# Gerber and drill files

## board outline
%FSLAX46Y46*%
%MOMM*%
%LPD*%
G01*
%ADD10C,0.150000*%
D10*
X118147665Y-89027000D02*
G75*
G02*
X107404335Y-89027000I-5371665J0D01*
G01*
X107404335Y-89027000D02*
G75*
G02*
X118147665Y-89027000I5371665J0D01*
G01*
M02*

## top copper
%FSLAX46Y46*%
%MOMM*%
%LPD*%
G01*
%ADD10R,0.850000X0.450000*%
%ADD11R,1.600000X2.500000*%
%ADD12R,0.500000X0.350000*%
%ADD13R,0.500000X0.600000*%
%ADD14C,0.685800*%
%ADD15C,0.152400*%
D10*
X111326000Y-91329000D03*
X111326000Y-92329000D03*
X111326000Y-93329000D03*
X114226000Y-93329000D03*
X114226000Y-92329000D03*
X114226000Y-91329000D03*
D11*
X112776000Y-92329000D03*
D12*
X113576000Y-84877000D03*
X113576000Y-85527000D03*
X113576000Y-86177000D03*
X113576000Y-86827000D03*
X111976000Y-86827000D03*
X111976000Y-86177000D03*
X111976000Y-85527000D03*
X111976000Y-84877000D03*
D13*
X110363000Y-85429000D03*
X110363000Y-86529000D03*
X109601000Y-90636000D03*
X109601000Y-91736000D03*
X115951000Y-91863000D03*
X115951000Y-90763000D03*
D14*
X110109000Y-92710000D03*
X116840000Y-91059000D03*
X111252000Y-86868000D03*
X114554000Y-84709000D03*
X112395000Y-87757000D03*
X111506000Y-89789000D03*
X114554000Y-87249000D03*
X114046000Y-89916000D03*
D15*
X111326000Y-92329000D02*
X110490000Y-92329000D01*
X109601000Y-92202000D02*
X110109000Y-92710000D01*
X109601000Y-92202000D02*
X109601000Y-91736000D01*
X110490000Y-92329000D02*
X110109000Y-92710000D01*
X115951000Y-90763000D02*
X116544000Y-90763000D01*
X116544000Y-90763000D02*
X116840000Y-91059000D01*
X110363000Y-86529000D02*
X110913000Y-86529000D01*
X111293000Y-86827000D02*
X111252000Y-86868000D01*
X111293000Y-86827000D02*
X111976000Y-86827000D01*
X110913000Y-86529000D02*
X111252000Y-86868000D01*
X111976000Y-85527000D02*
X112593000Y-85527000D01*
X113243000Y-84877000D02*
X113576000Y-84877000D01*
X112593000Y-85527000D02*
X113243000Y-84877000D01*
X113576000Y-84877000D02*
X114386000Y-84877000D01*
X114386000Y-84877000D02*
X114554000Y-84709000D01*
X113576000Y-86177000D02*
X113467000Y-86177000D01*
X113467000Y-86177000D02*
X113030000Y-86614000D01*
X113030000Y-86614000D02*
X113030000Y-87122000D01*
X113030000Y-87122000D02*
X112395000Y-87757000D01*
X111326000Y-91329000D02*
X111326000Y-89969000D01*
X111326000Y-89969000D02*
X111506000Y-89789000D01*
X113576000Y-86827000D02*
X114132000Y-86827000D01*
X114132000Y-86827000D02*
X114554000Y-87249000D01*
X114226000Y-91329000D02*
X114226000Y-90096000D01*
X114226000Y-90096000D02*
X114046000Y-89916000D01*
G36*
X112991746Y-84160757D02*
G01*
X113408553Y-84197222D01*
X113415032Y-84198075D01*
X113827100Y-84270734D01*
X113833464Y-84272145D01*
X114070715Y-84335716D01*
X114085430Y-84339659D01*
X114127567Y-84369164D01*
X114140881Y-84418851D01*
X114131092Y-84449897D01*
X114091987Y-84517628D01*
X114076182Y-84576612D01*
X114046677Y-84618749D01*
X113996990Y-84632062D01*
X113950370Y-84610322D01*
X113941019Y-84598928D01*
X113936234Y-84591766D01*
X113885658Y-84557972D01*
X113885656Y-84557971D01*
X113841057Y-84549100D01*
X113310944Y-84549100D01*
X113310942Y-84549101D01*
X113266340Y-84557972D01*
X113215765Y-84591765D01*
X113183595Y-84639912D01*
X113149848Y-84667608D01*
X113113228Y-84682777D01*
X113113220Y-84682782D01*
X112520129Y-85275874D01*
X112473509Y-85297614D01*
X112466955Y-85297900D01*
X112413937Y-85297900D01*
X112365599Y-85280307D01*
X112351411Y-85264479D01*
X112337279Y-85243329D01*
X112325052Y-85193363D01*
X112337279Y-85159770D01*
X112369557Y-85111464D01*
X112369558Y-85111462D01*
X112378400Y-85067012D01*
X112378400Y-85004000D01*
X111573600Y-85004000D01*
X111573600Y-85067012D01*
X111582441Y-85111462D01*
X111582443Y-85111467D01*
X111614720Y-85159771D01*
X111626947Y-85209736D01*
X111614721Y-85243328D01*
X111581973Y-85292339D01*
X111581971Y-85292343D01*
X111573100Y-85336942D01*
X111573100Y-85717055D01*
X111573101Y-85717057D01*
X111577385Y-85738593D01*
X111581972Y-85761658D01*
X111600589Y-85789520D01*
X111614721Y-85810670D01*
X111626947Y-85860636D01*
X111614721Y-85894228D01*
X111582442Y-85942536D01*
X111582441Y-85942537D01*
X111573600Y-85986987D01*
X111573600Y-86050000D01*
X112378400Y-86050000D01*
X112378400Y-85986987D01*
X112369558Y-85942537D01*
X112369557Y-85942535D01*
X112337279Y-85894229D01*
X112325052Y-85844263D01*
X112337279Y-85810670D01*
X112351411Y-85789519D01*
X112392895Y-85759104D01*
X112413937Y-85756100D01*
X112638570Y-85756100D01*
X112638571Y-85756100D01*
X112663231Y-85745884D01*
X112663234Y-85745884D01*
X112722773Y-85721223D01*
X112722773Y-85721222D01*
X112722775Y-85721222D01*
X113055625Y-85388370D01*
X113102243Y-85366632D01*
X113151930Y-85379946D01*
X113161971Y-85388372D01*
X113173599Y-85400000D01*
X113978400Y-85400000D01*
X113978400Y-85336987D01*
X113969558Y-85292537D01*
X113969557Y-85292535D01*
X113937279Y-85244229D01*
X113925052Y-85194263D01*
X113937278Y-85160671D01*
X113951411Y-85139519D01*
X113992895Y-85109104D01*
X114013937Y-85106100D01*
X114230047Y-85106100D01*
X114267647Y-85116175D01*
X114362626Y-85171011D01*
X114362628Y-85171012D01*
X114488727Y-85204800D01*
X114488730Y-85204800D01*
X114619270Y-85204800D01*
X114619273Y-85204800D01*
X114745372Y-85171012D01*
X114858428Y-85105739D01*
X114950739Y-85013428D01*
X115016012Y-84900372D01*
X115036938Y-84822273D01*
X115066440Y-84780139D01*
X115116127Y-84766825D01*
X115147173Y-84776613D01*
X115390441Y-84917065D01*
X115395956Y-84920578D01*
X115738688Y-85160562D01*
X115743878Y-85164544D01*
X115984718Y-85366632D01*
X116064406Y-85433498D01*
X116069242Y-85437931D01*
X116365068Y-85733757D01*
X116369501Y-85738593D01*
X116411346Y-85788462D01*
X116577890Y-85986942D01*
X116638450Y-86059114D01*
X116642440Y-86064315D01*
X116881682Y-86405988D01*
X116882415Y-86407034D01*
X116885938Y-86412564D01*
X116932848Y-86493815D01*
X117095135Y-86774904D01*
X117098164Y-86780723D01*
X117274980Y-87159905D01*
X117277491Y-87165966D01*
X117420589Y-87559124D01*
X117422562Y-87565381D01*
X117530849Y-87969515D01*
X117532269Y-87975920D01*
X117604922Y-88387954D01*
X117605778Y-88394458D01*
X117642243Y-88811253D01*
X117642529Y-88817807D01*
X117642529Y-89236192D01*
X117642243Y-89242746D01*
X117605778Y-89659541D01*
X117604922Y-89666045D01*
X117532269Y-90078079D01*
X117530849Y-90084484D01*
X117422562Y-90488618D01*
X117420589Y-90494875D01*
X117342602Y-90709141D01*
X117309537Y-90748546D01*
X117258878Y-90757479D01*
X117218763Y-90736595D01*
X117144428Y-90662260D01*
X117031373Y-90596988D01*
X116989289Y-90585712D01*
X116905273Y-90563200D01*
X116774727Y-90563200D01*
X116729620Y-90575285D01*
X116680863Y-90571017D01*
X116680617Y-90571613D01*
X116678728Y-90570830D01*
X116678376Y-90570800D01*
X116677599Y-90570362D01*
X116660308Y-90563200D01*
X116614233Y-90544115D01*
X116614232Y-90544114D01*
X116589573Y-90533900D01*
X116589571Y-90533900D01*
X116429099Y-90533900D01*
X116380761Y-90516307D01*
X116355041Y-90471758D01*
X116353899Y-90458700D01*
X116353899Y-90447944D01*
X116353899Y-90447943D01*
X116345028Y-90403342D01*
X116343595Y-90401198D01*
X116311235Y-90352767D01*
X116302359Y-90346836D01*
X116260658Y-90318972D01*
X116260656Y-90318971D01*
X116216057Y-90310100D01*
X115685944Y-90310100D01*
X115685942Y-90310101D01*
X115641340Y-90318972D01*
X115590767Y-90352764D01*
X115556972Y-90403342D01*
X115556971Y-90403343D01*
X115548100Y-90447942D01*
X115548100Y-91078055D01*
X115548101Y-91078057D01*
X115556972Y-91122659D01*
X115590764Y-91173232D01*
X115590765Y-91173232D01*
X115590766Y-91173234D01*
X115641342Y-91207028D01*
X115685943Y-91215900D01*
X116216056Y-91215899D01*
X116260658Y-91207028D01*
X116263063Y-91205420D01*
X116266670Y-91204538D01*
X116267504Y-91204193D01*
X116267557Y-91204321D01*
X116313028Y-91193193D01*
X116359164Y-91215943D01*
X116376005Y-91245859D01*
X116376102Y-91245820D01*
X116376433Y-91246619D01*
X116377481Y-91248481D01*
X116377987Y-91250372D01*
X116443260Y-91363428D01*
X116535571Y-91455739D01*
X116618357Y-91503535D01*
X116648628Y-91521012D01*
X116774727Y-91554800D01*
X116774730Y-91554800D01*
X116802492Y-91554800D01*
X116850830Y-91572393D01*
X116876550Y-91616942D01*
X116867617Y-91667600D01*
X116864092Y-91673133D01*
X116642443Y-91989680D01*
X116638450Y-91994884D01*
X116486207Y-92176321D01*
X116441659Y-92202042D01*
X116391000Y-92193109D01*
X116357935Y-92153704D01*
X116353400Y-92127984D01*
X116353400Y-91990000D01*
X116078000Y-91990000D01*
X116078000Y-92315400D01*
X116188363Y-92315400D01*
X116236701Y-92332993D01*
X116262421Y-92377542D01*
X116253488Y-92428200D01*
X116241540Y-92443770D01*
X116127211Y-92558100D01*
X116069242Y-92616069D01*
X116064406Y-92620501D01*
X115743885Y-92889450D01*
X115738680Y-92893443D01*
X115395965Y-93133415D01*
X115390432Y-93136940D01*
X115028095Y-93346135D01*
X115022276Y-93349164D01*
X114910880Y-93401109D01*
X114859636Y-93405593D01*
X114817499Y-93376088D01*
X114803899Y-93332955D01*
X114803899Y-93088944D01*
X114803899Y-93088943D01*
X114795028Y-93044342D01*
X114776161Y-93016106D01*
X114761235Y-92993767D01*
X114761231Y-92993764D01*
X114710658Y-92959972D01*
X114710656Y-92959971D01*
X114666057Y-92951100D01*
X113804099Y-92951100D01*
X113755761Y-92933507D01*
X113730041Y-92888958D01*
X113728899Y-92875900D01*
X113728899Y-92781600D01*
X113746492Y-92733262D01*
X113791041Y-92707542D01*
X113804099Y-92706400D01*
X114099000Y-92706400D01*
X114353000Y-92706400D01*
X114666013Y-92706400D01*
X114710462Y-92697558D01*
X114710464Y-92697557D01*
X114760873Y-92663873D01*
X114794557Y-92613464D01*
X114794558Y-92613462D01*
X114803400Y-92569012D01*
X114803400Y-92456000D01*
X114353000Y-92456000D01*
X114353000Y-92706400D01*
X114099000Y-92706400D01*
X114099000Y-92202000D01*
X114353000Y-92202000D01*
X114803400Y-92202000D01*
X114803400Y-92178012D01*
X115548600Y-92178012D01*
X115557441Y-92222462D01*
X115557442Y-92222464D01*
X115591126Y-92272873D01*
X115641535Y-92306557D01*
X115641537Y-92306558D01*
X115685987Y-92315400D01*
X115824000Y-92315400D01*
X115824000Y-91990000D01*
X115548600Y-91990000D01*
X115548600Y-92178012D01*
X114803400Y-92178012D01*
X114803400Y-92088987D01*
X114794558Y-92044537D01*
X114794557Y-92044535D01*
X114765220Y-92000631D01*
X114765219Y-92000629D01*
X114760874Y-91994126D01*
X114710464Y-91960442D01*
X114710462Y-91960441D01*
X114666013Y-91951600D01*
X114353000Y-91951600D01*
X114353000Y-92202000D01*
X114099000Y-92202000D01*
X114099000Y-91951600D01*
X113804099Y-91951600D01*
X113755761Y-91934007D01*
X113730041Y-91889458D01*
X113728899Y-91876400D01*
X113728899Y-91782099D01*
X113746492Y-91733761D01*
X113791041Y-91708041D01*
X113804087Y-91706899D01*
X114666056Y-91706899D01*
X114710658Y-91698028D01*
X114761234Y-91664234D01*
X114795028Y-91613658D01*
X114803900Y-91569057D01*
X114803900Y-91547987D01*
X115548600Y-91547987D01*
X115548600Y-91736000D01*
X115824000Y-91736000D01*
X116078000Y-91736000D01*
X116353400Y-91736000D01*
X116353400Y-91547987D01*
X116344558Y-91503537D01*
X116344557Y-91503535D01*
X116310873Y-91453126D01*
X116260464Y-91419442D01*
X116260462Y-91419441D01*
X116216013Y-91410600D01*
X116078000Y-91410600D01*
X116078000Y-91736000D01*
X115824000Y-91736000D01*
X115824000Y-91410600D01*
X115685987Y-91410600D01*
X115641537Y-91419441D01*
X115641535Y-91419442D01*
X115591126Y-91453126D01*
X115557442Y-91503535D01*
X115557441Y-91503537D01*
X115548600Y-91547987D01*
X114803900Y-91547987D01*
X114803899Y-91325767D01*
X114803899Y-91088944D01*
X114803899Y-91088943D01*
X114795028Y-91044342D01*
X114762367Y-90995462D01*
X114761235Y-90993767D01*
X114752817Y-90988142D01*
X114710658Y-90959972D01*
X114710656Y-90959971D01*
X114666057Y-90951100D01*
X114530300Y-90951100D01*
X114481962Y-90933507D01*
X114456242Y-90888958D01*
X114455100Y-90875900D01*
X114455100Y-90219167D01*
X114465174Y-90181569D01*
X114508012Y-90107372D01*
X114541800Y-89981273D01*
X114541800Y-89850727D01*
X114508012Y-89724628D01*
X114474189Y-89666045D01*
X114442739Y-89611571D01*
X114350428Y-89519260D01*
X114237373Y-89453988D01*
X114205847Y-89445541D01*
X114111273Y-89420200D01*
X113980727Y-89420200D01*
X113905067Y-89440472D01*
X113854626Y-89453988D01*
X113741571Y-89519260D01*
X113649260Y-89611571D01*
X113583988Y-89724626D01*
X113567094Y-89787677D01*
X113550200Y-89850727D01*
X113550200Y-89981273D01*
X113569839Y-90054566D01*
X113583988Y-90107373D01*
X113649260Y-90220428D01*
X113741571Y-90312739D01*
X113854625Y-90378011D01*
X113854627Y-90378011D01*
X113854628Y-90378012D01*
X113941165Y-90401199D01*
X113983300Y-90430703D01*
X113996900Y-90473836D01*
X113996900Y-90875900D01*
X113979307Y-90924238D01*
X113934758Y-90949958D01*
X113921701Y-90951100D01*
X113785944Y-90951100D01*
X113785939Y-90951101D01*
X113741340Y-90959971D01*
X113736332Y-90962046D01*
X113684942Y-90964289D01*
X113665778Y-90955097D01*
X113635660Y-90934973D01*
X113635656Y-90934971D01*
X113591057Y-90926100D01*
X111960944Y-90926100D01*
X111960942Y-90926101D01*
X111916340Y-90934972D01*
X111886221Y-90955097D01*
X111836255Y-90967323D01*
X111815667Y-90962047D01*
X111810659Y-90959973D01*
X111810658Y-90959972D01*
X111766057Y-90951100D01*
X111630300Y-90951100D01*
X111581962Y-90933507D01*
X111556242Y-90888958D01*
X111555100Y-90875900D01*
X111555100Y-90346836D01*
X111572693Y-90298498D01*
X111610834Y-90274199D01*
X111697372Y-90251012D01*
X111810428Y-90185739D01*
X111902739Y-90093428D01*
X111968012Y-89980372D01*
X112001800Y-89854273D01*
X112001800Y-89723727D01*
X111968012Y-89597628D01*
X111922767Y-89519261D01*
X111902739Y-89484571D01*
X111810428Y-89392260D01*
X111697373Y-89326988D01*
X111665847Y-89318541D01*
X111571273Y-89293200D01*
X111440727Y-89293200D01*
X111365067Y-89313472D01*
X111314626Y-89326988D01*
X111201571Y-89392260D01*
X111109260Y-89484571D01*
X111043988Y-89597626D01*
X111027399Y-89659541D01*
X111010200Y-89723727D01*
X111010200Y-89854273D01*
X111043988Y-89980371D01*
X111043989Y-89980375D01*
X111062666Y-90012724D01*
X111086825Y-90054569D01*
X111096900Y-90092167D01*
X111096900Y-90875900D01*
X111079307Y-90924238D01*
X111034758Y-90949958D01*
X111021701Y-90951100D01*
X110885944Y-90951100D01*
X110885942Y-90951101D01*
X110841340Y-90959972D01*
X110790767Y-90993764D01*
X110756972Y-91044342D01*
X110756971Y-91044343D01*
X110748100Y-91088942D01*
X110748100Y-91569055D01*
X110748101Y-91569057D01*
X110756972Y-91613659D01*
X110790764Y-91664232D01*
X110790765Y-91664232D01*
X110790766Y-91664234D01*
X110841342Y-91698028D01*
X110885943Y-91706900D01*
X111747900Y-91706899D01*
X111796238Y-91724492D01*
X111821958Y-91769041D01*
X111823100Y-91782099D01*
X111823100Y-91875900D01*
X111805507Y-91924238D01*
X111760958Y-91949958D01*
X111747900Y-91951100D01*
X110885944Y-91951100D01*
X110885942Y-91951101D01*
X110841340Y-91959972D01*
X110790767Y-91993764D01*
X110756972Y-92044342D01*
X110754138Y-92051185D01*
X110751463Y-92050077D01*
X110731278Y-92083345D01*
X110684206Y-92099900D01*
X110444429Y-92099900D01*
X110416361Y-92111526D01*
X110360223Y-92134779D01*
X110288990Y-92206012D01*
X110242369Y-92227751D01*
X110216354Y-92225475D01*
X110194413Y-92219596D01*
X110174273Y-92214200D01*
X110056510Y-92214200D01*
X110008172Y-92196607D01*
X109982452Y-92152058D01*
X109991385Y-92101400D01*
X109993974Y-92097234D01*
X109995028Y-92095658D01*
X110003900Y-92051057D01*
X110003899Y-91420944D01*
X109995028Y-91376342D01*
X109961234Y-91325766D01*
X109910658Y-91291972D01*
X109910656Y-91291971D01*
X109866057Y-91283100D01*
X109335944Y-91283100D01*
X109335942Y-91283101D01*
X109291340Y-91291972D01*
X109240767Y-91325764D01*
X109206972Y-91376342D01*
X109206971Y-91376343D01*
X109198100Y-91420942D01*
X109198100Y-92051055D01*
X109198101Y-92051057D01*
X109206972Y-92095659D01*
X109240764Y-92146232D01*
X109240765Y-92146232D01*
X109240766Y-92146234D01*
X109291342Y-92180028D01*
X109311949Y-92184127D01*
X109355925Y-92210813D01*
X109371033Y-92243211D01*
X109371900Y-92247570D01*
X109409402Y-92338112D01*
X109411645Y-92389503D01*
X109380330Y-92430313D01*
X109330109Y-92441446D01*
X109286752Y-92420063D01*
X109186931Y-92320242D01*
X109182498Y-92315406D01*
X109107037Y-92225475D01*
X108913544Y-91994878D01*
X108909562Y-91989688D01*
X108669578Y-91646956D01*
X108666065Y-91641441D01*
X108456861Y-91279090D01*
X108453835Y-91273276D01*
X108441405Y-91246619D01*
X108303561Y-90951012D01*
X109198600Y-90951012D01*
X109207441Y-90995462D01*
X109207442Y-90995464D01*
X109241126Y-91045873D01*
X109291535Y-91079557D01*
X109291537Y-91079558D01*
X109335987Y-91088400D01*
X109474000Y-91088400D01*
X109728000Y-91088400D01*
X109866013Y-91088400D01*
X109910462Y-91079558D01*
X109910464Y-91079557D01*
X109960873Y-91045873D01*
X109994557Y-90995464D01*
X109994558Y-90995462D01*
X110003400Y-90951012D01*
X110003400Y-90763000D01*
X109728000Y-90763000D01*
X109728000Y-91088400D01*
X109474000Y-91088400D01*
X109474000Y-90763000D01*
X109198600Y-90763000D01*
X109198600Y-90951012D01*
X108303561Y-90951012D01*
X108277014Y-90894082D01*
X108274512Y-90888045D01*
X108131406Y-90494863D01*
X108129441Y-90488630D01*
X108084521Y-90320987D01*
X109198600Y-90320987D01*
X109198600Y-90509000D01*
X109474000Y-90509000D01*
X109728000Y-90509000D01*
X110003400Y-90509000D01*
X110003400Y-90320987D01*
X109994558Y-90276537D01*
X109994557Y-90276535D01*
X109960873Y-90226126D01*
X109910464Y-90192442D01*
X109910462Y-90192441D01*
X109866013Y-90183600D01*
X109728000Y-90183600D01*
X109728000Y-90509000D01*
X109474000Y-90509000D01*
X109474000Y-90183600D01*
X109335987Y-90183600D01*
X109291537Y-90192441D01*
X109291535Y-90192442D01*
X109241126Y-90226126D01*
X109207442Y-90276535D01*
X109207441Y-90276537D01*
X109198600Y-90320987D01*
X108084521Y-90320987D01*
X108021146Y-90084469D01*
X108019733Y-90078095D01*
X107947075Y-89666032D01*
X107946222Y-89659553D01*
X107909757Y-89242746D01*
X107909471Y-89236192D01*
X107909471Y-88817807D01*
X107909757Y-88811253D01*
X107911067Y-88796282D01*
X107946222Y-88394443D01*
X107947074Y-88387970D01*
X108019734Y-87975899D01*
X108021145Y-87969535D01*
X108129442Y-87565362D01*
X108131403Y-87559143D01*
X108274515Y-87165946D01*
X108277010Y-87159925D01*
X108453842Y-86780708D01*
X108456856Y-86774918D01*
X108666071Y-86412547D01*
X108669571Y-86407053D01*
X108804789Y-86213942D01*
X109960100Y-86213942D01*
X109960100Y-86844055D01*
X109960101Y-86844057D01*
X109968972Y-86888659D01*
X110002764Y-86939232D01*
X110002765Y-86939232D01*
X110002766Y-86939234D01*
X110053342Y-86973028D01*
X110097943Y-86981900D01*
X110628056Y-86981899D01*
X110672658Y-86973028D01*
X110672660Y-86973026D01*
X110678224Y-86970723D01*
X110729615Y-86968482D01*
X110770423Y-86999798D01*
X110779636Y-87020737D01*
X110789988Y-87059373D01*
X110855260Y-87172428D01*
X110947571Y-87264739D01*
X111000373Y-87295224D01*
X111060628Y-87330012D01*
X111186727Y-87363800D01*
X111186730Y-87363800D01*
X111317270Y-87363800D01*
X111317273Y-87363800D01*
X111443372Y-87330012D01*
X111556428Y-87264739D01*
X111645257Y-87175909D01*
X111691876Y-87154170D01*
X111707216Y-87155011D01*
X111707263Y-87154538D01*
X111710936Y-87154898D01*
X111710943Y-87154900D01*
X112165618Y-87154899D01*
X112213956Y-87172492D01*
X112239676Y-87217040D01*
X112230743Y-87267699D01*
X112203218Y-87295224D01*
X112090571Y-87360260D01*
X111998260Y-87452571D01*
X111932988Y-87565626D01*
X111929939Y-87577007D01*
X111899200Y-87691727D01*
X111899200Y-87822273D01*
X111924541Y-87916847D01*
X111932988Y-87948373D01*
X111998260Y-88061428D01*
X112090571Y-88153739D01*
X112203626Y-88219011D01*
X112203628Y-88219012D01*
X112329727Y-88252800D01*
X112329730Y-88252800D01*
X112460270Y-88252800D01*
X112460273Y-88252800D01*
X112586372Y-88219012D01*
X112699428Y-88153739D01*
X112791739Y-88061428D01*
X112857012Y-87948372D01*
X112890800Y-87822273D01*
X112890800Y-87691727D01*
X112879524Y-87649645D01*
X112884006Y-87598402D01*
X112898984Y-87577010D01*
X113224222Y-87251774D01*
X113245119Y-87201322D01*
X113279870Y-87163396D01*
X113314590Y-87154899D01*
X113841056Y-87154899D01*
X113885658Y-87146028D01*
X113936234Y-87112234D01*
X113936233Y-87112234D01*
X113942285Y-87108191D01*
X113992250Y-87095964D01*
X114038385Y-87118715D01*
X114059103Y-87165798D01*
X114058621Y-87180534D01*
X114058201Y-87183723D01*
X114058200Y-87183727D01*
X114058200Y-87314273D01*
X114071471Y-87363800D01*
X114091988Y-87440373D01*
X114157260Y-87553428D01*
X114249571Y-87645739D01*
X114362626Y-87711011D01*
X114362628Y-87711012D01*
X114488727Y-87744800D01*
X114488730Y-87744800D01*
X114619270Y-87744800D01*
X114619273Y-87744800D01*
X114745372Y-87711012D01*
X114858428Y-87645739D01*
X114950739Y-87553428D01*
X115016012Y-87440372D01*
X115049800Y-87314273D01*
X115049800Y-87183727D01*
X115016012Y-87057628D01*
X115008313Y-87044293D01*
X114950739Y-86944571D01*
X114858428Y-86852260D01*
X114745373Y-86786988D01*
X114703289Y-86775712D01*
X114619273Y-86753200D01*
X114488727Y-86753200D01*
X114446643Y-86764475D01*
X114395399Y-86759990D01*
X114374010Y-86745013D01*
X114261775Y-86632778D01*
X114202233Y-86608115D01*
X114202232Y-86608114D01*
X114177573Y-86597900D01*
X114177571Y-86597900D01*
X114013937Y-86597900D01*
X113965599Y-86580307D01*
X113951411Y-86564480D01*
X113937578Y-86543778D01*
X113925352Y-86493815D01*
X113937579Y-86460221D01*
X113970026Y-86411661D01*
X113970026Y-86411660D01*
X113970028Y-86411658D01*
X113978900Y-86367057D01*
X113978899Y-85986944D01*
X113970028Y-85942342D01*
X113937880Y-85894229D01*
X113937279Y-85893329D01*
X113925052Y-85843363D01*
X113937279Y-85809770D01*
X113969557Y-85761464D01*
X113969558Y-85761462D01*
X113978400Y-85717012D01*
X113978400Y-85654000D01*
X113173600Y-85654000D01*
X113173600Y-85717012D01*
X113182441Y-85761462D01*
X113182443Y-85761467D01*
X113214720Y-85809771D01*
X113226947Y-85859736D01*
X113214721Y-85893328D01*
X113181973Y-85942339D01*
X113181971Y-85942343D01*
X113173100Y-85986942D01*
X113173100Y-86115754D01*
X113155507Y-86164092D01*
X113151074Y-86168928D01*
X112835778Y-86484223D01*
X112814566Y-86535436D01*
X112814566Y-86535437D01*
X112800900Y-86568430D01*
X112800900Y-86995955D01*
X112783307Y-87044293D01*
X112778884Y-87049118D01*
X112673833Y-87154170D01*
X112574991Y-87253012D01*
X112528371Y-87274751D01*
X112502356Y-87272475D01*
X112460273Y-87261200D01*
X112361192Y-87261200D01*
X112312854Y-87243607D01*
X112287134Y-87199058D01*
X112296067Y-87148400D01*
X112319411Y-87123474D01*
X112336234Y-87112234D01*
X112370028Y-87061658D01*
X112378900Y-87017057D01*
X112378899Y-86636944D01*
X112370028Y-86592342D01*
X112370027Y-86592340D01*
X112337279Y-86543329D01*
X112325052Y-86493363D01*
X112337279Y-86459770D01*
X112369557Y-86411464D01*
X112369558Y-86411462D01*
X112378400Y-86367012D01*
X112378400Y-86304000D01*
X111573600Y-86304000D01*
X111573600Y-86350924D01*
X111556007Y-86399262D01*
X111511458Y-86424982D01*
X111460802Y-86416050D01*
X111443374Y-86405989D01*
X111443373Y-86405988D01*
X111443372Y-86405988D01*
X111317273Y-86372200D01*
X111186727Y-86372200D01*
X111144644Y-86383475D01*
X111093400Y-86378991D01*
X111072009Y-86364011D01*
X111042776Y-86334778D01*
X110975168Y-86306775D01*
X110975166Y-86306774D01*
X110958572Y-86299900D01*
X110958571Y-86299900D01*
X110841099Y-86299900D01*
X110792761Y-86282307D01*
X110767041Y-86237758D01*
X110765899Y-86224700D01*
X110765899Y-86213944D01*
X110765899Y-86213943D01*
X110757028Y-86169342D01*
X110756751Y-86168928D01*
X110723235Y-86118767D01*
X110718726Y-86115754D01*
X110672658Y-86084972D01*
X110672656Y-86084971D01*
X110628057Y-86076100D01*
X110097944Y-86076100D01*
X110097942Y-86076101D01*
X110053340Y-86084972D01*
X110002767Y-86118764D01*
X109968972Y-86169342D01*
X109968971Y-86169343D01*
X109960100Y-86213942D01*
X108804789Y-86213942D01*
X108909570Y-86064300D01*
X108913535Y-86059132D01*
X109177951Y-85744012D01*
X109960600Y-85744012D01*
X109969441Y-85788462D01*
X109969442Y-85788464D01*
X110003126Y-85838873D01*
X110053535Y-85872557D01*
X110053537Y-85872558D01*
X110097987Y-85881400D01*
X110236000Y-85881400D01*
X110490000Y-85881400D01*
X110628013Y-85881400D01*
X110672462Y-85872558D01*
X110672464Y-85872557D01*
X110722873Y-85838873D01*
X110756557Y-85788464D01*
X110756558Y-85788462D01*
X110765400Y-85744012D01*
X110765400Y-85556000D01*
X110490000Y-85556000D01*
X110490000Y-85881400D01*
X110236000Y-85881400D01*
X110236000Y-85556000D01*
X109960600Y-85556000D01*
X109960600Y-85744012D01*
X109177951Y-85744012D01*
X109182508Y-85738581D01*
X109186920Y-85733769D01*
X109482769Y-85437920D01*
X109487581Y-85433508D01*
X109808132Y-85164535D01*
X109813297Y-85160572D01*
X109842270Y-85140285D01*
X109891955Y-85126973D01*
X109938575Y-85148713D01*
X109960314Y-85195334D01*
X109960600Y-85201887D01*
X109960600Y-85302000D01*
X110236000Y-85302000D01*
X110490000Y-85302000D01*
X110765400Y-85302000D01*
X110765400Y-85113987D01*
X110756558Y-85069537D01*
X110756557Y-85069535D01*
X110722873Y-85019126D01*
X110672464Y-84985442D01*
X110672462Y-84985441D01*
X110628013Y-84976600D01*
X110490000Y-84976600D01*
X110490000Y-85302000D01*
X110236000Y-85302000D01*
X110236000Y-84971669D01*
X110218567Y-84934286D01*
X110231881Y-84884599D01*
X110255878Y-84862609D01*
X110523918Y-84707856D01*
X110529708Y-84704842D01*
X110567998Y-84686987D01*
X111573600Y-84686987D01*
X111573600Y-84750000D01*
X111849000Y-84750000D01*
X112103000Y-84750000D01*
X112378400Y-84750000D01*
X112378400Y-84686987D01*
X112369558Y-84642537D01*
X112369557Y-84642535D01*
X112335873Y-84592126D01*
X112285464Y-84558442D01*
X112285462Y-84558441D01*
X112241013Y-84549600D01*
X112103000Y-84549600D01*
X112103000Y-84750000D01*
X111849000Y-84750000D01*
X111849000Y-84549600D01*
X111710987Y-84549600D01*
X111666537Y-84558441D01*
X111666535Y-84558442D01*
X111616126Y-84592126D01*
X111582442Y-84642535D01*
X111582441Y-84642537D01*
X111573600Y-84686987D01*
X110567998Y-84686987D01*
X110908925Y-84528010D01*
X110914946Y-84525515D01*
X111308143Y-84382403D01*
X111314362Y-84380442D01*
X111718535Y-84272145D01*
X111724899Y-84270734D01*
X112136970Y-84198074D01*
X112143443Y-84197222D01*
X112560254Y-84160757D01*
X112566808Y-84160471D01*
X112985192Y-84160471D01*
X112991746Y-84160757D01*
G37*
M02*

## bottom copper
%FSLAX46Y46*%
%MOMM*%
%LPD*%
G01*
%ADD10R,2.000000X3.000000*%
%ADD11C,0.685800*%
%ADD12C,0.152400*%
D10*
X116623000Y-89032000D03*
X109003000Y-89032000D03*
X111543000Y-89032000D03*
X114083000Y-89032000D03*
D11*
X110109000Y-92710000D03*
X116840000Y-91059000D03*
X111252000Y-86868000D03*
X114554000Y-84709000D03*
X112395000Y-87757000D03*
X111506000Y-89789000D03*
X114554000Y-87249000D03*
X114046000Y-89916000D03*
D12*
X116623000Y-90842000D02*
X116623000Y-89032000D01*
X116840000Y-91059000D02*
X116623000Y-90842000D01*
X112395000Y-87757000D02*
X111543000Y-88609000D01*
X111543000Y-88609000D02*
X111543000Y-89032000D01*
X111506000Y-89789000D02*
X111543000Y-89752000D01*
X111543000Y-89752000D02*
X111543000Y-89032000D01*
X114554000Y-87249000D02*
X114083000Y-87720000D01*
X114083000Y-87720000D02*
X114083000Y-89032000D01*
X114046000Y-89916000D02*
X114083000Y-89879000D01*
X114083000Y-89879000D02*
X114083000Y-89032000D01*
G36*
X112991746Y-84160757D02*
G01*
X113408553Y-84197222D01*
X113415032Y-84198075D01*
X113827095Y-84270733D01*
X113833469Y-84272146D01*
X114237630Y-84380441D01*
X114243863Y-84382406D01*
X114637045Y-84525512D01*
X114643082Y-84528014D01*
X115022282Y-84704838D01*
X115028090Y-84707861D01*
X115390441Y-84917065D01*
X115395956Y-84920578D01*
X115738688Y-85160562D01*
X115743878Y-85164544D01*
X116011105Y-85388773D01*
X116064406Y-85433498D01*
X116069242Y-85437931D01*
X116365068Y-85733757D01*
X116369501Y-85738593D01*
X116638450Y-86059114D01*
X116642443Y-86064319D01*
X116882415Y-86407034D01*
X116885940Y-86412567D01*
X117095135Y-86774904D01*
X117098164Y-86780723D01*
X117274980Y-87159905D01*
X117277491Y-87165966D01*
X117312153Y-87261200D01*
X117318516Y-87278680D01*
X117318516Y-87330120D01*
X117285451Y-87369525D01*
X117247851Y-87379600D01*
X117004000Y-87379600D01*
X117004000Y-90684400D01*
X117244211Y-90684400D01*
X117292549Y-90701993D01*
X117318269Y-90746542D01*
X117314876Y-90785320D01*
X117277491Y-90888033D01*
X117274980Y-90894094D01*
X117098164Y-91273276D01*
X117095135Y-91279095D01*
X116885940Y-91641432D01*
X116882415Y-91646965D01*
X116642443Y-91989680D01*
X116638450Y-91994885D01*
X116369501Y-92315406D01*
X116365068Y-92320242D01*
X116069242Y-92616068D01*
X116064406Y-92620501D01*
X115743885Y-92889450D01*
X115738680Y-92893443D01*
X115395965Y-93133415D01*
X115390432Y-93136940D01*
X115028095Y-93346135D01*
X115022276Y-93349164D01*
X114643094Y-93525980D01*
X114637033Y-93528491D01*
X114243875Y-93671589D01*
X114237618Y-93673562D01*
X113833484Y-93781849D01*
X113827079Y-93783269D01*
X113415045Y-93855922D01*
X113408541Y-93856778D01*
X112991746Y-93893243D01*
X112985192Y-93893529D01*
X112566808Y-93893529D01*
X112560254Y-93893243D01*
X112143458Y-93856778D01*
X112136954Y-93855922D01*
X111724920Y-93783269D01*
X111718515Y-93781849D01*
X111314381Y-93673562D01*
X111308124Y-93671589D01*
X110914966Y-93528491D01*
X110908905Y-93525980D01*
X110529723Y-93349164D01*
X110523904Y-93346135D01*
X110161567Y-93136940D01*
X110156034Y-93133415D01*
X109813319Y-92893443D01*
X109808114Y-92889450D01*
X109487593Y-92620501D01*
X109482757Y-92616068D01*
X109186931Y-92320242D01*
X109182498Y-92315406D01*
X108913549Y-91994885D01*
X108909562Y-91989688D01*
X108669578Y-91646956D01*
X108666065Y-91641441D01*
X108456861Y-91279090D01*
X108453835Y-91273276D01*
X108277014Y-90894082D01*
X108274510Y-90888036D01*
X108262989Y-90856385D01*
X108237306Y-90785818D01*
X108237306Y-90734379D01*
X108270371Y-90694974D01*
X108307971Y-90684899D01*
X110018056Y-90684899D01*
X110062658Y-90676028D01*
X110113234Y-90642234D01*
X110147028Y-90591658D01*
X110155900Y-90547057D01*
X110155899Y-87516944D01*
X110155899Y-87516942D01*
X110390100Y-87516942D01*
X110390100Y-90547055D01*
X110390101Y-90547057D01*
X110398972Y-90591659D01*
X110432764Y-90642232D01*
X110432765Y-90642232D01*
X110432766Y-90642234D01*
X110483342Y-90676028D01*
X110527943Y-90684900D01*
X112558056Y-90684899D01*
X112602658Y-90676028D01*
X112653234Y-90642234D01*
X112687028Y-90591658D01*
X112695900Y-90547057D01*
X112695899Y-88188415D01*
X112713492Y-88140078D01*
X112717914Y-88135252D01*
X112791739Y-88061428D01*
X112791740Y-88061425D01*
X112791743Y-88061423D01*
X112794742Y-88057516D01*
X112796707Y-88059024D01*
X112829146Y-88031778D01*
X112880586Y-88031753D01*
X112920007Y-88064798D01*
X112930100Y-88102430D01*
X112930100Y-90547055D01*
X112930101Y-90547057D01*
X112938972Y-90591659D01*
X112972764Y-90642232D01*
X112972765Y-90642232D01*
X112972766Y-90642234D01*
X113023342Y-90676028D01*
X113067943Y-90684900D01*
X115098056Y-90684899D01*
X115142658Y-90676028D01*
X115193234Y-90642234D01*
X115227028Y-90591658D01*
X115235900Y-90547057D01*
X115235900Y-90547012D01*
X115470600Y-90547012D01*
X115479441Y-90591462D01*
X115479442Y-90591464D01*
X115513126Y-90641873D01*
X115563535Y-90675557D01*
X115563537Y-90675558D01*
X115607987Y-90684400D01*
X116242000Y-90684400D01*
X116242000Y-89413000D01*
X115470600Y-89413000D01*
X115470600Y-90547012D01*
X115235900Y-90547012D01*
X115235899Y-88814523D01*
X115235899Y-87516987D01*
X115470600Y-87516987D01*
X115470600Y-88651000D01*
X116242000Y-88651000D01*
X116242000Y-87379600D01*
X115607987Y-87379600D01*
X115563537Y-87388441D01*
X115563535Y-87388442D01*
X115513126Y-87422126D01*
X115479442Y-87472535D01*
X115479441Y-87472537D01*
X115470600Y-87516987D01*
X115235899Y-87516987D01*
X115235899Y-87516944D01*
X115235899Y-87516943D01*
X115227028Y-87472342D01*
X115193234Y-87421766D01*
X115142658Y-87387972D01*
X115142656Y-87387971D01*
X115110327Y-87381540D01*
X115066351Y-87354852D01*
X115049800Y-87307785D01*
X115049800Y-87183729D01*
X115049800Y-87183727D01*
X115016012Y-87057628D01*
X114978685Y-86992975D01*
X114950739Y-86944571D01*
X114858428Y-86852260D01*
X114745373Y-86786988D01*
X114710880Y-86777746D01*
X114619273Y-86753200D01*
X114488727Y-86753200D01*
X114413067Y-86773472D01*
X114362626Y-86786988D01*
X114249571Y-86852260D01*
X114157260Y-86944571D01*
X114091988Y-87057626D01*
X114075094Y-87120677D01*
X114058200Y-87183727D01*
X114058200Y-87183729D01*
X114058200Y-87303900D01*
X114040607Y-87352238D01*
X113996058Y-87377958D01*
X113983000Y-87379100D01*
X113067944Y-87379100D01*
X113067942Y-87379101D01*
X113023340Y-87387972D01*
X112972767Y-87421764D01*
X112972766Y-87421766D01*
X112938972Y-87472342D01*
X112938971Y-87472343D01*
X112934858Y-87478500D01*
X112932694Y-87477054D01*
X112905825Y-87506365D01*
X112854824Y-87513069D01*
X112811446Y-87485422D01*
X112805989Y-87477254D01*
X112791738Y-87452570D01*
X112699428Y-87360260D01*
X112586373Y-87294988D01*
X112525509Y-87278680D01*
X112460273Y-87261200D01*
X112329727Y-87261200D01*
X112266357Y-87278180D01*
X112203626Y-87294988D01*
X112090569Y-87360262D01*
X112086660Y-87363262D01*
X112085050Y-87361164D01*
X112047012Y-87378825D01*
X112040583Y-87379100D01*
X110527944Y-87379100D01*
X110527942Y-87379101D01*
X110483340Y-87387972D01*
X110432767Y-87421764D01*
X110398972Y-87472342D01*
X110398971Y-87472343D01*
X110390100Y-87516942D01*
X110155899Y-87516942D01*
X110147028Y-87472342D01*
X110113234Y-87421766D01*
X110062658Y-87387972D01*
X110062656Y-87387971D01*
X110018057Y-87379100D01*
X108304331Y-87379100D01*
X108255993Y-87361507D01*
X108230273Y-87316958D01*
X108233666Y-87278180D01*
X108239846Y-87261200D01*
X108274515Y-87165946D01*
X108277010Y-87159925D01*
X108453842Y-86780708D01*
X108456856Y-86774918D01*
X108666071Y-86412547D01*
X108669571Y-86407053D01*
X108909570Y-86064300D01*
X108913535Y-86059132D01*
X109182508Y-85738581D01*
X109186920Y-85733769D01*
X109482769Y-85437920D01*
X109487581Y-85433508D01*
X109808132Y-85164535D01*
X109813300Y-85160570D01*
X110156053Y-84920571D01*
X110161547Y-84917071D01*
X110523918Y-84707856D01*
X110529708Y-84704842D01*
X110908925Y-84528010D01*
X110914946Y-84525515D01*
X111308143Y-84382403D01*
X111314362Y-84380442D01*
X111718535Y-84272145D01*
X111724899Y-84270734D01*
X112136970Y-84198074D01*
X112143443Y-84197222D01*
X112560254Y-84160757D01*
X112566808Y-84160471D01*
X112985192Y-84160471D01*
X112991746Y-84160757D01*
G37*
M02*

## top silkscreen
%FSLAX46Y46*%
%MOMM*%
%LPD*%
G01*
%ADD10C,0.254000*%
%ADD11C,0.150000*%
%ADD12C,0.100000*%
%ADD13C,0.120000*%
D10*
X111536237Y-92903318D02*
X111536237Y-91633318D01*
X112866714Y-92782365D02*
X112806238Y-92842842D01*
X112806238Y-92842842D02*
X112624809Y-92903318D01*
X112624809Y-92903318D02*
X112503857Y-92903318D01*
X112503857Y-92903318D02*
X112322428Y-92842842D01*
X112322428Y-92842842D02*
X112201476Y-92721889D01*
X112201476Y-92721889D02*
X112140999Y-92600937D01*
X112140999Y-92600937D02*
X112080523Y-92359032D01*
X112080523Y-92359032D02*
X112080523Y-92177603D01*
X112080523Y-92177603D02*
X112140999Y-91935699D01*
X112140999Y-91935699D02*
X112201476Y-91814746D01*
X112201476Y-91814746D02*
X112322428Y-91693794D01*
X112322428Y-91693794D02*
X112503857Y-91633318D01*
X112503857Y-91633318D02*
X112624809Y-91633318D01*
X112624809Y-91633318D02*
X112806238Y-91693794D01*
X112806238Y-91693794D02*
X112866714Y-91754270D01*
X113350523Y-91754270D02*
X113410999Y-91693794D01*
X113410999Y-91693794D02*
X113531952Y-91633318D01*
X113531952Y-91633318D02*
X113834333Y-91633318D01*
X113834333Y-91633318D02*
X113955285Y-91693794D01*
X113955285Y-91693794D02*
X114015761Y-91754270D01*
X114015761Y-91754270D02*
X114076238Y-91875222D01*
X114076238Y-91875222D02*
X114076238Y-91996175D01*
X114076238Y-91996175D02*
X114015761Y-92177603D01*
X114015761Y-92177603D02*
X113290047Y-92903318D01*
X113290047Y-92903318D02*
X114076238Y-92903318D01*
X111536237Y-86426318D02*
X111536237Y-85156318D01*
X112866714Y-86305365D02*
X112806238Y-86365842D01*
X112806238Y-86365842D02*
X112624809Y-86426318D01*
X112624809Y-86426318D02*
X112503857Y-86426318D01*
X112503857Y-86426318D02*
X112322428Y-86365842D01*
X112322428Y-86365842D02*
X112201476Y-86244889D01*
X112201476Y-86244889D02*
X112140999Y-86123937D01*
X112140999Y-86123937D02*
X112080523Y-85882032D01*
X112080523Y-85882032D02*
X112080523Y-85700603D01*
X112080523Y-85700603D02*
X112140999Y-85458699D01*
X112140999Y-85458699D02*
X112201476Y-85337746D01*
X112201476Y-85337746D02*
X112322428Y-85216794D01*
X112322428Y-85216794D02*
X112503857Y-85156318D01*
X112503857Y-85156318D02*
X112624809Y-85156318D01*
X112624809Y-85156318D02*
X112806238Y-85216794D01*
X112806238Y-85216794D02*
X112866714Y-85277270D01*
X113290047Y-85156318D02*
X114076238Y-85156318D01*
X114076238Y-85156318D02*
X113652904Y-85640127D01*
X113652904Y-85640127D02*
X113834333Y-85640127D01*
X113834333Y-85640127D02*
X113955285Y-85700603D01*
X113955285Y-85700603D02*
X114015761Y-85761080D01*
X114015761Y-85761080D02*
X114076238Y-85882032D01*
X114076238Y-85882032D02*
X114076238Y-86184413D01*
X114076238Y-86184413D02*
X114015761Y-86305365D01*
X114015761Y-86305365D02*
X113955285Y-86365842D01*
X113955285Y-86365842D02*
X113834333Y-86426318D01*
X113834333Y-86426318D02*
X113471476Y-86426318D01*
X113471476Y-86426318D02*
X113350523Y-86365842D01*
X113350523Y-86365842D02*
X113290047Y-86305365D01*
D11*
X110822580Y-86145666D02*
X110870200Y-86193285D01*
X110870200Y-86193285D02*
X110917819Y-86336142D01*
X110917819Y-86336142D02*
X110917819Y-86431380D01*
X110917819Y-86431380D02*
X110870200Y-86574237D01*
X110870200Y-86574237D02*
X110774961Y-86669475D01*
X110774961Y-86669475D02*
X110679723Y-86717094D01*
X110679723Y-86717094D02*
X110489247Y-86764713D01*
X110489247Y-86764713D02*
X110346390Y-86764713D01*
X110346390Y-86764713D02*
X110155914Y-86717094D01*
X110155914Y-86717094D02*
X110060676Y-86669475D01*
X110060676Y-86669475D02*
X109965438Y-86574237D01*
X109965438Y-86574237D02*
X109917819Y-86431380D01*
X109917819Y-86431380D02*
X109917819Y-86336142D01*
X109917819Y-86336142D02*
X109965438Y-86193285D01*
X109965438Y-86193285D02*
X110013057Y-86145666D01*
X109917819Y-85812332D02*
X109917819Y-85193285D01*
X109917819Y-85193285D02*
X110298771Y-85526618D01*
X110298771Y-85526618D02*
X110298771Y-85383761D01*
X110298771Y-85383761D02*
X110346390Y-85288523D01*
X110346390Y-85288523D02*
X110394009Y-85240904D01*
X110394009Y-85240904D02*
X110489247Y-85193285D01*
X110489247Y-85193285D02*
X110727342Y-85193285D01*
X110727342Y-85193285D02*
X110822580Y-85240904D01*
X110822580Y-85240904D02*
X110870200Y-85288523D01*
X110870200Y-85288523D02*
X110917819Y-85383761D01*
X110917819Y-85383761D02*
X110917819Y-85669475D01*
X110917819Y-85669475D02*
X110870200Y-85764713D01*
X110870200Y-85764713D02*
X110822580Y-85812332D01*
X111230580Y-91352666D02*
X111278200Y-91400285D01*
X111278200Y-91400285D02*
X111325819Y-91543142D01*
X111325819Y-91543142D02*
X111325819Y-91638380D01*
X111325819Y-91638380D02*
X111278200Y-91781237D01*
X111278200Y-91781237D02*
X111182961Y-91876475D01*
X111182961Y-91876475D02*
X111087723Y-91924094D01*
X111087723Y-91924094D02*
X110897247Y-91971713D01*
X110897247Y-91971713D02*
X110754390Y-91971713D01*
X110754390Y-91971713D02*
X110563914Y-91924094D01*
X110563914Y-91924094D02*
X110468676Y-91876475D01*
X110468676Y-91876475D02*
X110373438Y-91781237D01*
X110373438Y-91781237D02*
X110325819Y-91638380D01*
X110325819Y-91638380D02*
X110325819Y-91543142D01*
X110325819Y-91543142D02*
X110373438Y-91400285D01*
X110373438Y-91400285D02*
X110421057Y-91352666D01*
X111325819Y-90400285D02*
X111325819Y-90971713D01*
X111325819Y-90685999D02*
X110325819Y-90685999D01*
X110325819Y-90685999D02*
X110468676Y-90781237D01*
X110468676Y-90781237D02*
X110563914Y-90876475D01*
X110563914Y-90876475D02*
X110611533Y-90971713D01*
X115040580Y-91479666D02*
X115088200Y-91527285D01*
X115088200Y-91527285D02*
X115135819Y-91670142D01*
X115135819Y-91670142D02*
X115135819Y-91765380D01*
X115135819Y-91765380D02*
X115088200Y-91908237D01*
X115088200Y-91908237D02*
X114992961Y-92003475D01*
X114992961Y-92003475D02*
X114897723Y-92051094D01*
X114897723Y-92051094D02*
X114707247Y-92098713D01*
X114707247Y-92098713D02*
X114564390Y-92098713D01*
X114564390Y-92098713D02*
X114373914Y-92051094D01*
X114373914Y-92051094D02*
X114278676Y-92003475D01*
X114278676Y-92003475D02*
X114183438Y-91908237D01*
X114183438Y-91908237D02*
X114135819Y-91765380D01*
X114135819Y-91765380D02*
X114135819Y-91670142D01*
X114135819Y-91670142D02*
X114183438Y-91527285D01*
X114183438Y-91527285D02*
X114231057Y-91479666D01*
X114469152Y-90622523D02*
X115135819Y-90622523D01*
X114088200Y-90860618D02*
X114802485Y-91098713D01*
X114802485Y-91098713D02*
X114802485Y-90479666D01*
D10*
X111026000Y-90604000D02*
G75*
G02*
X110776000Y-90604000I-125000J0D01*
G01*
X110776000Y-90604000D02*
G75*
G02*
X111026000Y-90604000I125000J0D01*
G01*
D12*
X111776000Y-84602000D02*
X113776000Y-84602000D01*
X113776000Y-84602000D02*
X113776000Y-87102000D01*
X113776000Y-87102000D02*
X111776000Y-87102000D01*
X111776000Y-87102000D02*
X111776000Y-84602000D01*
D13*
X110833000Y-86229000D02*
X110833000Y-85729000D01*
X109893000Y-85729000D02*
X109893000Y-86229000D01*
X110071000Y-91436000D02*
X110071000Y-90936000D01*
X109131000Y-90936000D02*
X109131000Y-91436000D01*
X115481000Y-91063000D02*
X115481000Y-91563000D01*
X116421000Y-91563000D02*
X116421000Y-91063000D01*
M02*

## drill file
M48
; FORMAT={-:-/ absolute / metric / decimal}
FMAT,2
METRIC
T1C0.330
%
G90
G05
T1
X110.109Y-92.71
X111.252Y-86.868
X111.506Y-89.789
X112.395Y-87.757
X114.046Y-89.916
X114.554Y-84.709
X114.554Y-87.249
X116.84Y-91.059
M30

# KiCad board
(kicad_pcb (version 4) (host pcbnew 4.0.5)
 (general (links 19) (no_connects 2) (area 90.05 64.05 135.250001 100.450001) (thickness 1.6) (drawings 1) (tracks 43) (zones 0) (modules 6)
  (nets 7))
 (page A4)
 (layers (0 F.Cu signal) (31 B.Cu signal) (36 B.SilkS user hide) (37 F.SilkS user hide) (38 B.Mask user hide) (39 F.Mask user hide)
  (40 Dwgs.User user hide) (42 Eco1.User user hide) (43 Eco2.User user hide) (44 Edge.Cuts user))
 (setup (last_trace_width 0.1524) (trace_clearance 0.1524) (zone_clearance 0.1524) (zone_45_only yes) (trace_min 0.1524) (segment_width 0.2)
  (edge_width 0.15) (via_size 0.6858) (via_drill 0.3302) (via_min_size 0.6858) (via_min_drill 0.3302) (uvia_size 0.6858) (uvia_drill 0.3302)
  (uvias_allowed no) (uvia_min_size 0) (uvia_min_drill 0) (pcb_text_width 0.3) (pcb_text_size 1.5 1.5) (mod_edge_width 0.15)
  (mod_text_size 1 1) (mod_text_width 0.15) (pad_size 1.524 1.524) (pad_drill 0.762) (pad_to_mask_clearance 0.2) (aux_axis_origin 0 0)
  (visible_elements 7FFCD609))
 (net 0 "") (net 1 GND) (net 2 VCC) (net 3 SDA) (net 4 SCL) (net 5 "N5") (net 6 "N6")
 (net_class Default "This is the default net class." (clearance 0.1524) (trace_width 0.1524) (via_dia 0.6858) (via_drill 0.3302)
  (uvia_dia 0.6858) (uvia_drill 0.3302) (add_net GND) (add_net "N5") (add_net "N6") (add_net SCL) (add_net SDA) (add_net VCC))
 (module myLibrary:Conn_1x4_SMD (layer B.Cu) (at 112.903 90.932)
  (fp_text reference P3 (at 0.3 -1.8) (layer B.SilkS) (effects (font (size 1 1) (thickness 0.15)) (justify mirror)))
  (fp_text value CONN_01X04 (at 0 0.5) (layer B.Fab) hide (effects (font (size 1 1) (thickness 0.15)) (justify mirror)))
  (pad 4 smd rect (at 3.72 -1.9) (size 2 3) (layers B.Cu B.Mask) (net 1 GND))
  (pad 1 smd rect (at -3.9 -1.9) (size 2 3) (layers B.Cu B.Mask) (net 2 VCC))
  (pad 2 smd rect (at -1.36 -1.9) (size 2 3) (layers B.Cu B.Mask) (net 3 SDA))
  (pad 3 smd rect (at 1.18 -1.9) (size 2 3) (layers B.Cu B.Mask) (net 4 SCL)))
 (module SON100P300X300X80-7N (layer F.Cu) (at 112.776 92.329)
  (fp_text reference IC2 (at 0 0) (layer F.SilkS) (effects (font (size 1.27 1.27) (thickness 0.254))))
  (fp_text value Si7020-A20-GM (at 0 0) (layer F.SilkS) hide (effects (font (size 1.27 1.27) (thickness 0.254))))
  (fp_circle (center -1.875 -1.725) (end -1.75 -1.725) (layer F.SilkS) (width 0.254))
  (pad 1 smd rect (at -1.45 -1 90) (size 0.45 0.85) (layers F.Cu F.Mask) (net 3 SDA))
  (pad 2 smd rect (at -1.45 0 90) (size 0.45 0.85) (layers F.Cu F.Mask) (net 1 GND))
  (pad 3 smd rect (at -1.45 1 90) (size 0.45 0.85) (layers F.Cu F.Mask) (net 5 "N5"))
  (pad 4 smd rect (at 1.45 1 90) (size 0.45 0.85) (layers F.Cu F.Mask) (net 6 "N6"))
  (pad 5 smd rect (at 1.45 0 90) (size 0.45 0.85) (layers F.Cu F.Mask) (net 2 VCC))
  (pad 6 smd rect (at 1.45 -1 90) (size 0.45 0.85) (layers F.Cu F.Mask) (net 4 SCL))
  (pad 7 smd rect (at 0 0) (size 1.6 2.5) (layers F.Cu F.Mask) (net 1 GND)))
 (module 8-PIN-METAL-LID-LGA (layer F.Cu) (at 112.776 85.852)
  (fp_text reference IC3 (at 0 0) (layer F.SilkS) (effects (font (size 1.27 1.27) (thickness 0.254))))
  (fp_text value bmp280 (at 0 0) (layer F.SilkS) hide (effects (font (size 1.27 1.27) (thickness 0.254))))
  (fp_line (start -1 -1.25) (end 1 -1.25) (layer F.SilkS) (width 0.1))
  (fp_line (start 1 -1.25) (end 1 1.25) (layer F.SilkS) (width 0.1))
  (fp_line (start 1 1.25) (end -1 1.25) (layer F.SilkS) (width 0.1))
  (fp_line (start -1 1.25) (end -1 -1.25) (layer F.SilkS) (width 0.1))
  (pad 1 smd rect (at 0.8 -0.975 90) (size 0.35 0.5) (layers F.Cu F.Mask) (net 1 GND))
  (pad 2 smd rect (at 0.8 -0.325 90) (size 0.35 0.5) (layers F.Cu F.Mask) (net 2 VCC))
  (pad 3 smd rect (at 0.8 0.325 90) (size 0.35 0.5) (layers F.Cu F.Mask) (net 3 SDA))
  (pad 4 smd rect (at 0.8 0.975 90) (size 0.35 0.5) (layers F.Cu F.Mask) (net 4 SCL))
  (pad 5 smd rect (at -0.8 0.975 90) (size 0.35 0.5) (layers F.Cu F.Mask) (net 1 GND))
  (pad 6 smd rect (at -0.8 0.325 90) (size 0.35 0.5) (layers F.Cu F.Mask) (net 2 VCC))
  (pad 7 smd rect (at -0.8 -0.325 90) (size 0.35 0.5) (layers F.Cu F.Mask) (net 1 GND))
  (pad 8 smd rect (at -0.8 -0.975 90) (size 0.35 0.5) (layers F.Cu F.Mask) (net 2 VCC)))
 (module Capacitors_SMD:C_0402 (layer F.Cu) (at 110.363 85.979 270)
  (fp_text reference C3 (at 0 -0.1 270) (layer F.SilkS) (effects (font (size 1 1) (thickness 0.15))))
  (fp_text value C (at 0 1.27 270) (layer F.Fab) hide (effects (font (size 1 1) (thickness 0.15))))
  (fp_line (start 0.25 -0.47) (end -0.25 -0.47) (layer F.SilkS) (width 0.12))
  (fp_line (start -0.25 0.47) (end 0.25 0.47) (layer F.SilkS) (width 0.12))
  (pad 1 smd rect (at -0.55 0 270) (size 0.6 0.5) (layers F.Cu F.Mask) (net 2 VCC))
  (pad 2 smd rect (at 0.55 0 270) (size 0.6 0.5) (layers F.Cu F.Mask) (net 1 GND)))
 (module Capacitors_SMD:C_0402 (layer F.Cu) (at 109.601 91.186 270)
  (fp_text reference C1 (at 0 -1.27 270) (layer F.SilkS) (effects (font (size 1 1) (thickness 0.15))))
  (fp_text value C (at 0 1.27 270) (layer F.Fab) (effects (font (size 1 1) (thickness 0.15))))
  (fp_line (start 0.25 -0.47) (end -0.25 -0.47) (layer F.SilkS) (width 0.12))
  (fp_line (start -0.25 0.47) (end 0.25 0.47) (layer F.SilkS) (width 0.12))
  (pad 1 smd rect (at -0.55 0 270) (size 0.6 0.5) (layers F.Cu F.Mask) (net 2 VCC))
  (pad 2 smd rect (at 0.55 0 270) (size 0.6 0.5) (layers F.Cu F.Mask) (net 1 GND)))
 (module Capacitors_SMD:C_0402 (layer F.Cu) (at 115.951 91.313 90)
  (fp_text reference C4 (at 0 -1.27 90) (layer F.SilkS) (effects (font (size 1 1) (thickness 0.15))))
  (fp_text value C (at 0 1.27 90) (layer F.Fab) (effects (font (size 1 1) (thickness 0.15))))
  (fp_line (start 0.25 -0.47) (end -0.25 -0.47) (layer F.SilkS) (width 0.12))
  (fp_line (start -0.25 0.47) (end 0.25 0.47) (layer F.SilkS) (width 0.12))
  (pad 1 smd rect (at -0.55 0 90) (size 0.6 0.5) (layers F.Cu F.Mask) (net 2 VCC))
  (pad 2 smd rect (at 0.55 0 90) (size 0.6 0.5) (layers F.Cu F.Mask) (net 1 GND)))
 (gr_circle (center 112.776 89.027) (end 118.11 88.392) (layer Edge.Cuts) (width 0.15))
 (segment (start 111.326 92.329) (end 110.49 92.329) (width 0.1524) (layer F.Cu) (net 1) (status 400000))
 (segment (start 109.601 92.202) (end 110.109 92.71) (width 0.1524) (layer F.Cu) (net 1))
 (via (at 110.109 92.71) (size 0.6858) (drill 0.3302) (layers F.Cu B.Cu) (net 1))
 (segment (start 109.601 92.202) (end 109.601 91.736) (width 0.1524) (layer F.Cu) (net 1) (status 800000))
 (segment (start 110.49 92.329) (end 110.109 92.71) (width 0.1524) (layer F.Cu) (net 1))
 (segment (start 115.951 90.763) (end 116.544 90.763) (width 0.1524) (layer F.Cu) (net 1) (status 400000))
 (segment (start 116.623 90.842) (end 116.623 89.032) (width 0.1524) (layer B.Cu) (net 1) (status 800000))
 (segment (start 116.84 91.059) (end 116.623 90.842) (width 0.1524) (layer B.Cu) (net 1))
 (via (at 116.84 91.059) (size 0.6858) (drill 0.3302) (layers F.Cu B.Cu) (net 1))
 (segment (start 116.544 90.763) (end 116.84 91.059) (width 0.1524) (layer F.Cu) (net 1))
 (segment (start 110.363 86.529) (end 110.913 86.529) (width 0.1524) (layer F.Cu) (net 1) (status 400000))
 (segment (start 111.293 86.827) (end 111.252 86.868) (width 0.1524) (layer F.Cu) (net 1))
 (via (at 111.252 86.868) (size 0.6858) (drill 0.3302) (layers F.Cu B.Cu) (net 1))
 (segment (start 111.293 86.827) (end 111.976 86.827) (width 0.1524) (layer F.Cu) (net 1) (status 800000))
 (segment (start 110.913 86.529) (end 111.252 86.868) (width 0.1524) (layer F.Cu) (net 1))
 (segment (start 111.976 85.527) (end 112.593 85.527) (width 0.1524) (layer F.Cu) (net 1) (status 400000))
 (segment (start 113.243 84.877) (end 113.576 84.877) (width 0.1524) (layer F.Cu) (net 1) (status 800000))
 (segment (start 112.593 85.527) (end 113.243 84.877) (width 0.1524) (layer F.Cu) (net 1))
 (segment (start 113.576 84.877) (end 114.386 84.877) (width 0.1524) (layer F.Cu) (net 1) (status 400000))
 (via (at 114.554 84.709) (size 0.6858) (drill 0.3302) (layers F.Cu B.Cu) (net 1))
 (segment (start 114.386 84.877) (end 114.554 84.709) (width 0.1524) (layer F.Cu) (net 1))
 (segment (start 113.576 86.177) (end 113.467 86.177) (width 0.1524) (layer F.Cu) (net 3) (status C00000))
 (segment (start 113.467 86.177) (end 113.03 86.614) (width 0.1524) (layer F.Cu) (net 3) (status 400000))
 (segment (start 113.03 86.614) (end 113.03 87.122) (width 0.1524) (layer F.Cu) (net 3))
 (segment (start 113.03 87.122) (end 112.395 87.757) (width 0.1524) (layer F.Cu) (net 3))
 (via (at 112.395 87.757) (size 0.6858) (drill 0.3302) (layers F.Cu B.Cu) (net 3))
 (segment (start 112.395 87.757) (end 111.543 88.609) (width 0.1524) (layer B.Cu) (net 3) (status 800000))
 (segment (start 111.543 88.609) (end 111.543 89.032) (width 0.1524) (layer B.Cu) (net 3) (status C00000))
 (segment (start 111.326 91.329) (end 111.326 89.969) (width 0.1524) (layer F.Cu) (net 3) (status 400000))
 (segment (start 111.506 89.789) (end 111.543 89.752) (width 0.1524) (layer B.Cu) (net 3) (status 800000))
 (via (at 111.506 89.789) (size 0.6858) (drill 0.3302) (layers F.Cu B.Cu) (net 3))
 (segment (start 111.326 89.969) (end 111.506 89.789) (width 0.1524) (layer F.Cu) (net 3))
 (segment (start 111.543 89.752) (end 111.543 89.032) (width 0.1524) (layer B.Cu) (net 3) (status C00000))
 (segment (start 113.576 86.827) (end 114.132 86.827) (width 0.1524) (layer F.Cu) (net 4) (status 400000))
 (segment (start 114.554 87.249) (end 114.083 87.72) (width 0.1524) (layer B.Cu) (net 4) (status 800000))
 (via (at 114.554 87.249) (size 0.6858) (drill 0.3302) (layers F.Cu B.Cu) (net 4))
 (segment (start 114.132 86.827) (end 114.554 87.249) (width 0.1524) (layer F.Cu) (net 4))
 (segment (start 114.083 87.72) (end 114.083 89.032) (width 0.1524) (layer B.Cu) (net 4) (status C00000))
 (segment (start 114.226 91.329) (end 114.226 90.096) (width 0.1524) (layer F.Cu) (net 4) (status 400000))
 (segment (start 114.046 89.916) (end 114.083 89.879) (width 0.1524) (layer B.Cu) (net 4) (status 800000))
 (via (at 114.046 89.916) (size 0.6858) (drill 0.3302) (layers F.Cu B.Cu) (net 4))
 (segment (start 114.226 90.096) (end 114.046 89.916) (width 0.1524) (layer F.Cu) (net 4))
 (segment (start 114.083 89.879) (end 114.083 89.032) (width 0.1524) (layer B.Cu) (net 4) (status C00000))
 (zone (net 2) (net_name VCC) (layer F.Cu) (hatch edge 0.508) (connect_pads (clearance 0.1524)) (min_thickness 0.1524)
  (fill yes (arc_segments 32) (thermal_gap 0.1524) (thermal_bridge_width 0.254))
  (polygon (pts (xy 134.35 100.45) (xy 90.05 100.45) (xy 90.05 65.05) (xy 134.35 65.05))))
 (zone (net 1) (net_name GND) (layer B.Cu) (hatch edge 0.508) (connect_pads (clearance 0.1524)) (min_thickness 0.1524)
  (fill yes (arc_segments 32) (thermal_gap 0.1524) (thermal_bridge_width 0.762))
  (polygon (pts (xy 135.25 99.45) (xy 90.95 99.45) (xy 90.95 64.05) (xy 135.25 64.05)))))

